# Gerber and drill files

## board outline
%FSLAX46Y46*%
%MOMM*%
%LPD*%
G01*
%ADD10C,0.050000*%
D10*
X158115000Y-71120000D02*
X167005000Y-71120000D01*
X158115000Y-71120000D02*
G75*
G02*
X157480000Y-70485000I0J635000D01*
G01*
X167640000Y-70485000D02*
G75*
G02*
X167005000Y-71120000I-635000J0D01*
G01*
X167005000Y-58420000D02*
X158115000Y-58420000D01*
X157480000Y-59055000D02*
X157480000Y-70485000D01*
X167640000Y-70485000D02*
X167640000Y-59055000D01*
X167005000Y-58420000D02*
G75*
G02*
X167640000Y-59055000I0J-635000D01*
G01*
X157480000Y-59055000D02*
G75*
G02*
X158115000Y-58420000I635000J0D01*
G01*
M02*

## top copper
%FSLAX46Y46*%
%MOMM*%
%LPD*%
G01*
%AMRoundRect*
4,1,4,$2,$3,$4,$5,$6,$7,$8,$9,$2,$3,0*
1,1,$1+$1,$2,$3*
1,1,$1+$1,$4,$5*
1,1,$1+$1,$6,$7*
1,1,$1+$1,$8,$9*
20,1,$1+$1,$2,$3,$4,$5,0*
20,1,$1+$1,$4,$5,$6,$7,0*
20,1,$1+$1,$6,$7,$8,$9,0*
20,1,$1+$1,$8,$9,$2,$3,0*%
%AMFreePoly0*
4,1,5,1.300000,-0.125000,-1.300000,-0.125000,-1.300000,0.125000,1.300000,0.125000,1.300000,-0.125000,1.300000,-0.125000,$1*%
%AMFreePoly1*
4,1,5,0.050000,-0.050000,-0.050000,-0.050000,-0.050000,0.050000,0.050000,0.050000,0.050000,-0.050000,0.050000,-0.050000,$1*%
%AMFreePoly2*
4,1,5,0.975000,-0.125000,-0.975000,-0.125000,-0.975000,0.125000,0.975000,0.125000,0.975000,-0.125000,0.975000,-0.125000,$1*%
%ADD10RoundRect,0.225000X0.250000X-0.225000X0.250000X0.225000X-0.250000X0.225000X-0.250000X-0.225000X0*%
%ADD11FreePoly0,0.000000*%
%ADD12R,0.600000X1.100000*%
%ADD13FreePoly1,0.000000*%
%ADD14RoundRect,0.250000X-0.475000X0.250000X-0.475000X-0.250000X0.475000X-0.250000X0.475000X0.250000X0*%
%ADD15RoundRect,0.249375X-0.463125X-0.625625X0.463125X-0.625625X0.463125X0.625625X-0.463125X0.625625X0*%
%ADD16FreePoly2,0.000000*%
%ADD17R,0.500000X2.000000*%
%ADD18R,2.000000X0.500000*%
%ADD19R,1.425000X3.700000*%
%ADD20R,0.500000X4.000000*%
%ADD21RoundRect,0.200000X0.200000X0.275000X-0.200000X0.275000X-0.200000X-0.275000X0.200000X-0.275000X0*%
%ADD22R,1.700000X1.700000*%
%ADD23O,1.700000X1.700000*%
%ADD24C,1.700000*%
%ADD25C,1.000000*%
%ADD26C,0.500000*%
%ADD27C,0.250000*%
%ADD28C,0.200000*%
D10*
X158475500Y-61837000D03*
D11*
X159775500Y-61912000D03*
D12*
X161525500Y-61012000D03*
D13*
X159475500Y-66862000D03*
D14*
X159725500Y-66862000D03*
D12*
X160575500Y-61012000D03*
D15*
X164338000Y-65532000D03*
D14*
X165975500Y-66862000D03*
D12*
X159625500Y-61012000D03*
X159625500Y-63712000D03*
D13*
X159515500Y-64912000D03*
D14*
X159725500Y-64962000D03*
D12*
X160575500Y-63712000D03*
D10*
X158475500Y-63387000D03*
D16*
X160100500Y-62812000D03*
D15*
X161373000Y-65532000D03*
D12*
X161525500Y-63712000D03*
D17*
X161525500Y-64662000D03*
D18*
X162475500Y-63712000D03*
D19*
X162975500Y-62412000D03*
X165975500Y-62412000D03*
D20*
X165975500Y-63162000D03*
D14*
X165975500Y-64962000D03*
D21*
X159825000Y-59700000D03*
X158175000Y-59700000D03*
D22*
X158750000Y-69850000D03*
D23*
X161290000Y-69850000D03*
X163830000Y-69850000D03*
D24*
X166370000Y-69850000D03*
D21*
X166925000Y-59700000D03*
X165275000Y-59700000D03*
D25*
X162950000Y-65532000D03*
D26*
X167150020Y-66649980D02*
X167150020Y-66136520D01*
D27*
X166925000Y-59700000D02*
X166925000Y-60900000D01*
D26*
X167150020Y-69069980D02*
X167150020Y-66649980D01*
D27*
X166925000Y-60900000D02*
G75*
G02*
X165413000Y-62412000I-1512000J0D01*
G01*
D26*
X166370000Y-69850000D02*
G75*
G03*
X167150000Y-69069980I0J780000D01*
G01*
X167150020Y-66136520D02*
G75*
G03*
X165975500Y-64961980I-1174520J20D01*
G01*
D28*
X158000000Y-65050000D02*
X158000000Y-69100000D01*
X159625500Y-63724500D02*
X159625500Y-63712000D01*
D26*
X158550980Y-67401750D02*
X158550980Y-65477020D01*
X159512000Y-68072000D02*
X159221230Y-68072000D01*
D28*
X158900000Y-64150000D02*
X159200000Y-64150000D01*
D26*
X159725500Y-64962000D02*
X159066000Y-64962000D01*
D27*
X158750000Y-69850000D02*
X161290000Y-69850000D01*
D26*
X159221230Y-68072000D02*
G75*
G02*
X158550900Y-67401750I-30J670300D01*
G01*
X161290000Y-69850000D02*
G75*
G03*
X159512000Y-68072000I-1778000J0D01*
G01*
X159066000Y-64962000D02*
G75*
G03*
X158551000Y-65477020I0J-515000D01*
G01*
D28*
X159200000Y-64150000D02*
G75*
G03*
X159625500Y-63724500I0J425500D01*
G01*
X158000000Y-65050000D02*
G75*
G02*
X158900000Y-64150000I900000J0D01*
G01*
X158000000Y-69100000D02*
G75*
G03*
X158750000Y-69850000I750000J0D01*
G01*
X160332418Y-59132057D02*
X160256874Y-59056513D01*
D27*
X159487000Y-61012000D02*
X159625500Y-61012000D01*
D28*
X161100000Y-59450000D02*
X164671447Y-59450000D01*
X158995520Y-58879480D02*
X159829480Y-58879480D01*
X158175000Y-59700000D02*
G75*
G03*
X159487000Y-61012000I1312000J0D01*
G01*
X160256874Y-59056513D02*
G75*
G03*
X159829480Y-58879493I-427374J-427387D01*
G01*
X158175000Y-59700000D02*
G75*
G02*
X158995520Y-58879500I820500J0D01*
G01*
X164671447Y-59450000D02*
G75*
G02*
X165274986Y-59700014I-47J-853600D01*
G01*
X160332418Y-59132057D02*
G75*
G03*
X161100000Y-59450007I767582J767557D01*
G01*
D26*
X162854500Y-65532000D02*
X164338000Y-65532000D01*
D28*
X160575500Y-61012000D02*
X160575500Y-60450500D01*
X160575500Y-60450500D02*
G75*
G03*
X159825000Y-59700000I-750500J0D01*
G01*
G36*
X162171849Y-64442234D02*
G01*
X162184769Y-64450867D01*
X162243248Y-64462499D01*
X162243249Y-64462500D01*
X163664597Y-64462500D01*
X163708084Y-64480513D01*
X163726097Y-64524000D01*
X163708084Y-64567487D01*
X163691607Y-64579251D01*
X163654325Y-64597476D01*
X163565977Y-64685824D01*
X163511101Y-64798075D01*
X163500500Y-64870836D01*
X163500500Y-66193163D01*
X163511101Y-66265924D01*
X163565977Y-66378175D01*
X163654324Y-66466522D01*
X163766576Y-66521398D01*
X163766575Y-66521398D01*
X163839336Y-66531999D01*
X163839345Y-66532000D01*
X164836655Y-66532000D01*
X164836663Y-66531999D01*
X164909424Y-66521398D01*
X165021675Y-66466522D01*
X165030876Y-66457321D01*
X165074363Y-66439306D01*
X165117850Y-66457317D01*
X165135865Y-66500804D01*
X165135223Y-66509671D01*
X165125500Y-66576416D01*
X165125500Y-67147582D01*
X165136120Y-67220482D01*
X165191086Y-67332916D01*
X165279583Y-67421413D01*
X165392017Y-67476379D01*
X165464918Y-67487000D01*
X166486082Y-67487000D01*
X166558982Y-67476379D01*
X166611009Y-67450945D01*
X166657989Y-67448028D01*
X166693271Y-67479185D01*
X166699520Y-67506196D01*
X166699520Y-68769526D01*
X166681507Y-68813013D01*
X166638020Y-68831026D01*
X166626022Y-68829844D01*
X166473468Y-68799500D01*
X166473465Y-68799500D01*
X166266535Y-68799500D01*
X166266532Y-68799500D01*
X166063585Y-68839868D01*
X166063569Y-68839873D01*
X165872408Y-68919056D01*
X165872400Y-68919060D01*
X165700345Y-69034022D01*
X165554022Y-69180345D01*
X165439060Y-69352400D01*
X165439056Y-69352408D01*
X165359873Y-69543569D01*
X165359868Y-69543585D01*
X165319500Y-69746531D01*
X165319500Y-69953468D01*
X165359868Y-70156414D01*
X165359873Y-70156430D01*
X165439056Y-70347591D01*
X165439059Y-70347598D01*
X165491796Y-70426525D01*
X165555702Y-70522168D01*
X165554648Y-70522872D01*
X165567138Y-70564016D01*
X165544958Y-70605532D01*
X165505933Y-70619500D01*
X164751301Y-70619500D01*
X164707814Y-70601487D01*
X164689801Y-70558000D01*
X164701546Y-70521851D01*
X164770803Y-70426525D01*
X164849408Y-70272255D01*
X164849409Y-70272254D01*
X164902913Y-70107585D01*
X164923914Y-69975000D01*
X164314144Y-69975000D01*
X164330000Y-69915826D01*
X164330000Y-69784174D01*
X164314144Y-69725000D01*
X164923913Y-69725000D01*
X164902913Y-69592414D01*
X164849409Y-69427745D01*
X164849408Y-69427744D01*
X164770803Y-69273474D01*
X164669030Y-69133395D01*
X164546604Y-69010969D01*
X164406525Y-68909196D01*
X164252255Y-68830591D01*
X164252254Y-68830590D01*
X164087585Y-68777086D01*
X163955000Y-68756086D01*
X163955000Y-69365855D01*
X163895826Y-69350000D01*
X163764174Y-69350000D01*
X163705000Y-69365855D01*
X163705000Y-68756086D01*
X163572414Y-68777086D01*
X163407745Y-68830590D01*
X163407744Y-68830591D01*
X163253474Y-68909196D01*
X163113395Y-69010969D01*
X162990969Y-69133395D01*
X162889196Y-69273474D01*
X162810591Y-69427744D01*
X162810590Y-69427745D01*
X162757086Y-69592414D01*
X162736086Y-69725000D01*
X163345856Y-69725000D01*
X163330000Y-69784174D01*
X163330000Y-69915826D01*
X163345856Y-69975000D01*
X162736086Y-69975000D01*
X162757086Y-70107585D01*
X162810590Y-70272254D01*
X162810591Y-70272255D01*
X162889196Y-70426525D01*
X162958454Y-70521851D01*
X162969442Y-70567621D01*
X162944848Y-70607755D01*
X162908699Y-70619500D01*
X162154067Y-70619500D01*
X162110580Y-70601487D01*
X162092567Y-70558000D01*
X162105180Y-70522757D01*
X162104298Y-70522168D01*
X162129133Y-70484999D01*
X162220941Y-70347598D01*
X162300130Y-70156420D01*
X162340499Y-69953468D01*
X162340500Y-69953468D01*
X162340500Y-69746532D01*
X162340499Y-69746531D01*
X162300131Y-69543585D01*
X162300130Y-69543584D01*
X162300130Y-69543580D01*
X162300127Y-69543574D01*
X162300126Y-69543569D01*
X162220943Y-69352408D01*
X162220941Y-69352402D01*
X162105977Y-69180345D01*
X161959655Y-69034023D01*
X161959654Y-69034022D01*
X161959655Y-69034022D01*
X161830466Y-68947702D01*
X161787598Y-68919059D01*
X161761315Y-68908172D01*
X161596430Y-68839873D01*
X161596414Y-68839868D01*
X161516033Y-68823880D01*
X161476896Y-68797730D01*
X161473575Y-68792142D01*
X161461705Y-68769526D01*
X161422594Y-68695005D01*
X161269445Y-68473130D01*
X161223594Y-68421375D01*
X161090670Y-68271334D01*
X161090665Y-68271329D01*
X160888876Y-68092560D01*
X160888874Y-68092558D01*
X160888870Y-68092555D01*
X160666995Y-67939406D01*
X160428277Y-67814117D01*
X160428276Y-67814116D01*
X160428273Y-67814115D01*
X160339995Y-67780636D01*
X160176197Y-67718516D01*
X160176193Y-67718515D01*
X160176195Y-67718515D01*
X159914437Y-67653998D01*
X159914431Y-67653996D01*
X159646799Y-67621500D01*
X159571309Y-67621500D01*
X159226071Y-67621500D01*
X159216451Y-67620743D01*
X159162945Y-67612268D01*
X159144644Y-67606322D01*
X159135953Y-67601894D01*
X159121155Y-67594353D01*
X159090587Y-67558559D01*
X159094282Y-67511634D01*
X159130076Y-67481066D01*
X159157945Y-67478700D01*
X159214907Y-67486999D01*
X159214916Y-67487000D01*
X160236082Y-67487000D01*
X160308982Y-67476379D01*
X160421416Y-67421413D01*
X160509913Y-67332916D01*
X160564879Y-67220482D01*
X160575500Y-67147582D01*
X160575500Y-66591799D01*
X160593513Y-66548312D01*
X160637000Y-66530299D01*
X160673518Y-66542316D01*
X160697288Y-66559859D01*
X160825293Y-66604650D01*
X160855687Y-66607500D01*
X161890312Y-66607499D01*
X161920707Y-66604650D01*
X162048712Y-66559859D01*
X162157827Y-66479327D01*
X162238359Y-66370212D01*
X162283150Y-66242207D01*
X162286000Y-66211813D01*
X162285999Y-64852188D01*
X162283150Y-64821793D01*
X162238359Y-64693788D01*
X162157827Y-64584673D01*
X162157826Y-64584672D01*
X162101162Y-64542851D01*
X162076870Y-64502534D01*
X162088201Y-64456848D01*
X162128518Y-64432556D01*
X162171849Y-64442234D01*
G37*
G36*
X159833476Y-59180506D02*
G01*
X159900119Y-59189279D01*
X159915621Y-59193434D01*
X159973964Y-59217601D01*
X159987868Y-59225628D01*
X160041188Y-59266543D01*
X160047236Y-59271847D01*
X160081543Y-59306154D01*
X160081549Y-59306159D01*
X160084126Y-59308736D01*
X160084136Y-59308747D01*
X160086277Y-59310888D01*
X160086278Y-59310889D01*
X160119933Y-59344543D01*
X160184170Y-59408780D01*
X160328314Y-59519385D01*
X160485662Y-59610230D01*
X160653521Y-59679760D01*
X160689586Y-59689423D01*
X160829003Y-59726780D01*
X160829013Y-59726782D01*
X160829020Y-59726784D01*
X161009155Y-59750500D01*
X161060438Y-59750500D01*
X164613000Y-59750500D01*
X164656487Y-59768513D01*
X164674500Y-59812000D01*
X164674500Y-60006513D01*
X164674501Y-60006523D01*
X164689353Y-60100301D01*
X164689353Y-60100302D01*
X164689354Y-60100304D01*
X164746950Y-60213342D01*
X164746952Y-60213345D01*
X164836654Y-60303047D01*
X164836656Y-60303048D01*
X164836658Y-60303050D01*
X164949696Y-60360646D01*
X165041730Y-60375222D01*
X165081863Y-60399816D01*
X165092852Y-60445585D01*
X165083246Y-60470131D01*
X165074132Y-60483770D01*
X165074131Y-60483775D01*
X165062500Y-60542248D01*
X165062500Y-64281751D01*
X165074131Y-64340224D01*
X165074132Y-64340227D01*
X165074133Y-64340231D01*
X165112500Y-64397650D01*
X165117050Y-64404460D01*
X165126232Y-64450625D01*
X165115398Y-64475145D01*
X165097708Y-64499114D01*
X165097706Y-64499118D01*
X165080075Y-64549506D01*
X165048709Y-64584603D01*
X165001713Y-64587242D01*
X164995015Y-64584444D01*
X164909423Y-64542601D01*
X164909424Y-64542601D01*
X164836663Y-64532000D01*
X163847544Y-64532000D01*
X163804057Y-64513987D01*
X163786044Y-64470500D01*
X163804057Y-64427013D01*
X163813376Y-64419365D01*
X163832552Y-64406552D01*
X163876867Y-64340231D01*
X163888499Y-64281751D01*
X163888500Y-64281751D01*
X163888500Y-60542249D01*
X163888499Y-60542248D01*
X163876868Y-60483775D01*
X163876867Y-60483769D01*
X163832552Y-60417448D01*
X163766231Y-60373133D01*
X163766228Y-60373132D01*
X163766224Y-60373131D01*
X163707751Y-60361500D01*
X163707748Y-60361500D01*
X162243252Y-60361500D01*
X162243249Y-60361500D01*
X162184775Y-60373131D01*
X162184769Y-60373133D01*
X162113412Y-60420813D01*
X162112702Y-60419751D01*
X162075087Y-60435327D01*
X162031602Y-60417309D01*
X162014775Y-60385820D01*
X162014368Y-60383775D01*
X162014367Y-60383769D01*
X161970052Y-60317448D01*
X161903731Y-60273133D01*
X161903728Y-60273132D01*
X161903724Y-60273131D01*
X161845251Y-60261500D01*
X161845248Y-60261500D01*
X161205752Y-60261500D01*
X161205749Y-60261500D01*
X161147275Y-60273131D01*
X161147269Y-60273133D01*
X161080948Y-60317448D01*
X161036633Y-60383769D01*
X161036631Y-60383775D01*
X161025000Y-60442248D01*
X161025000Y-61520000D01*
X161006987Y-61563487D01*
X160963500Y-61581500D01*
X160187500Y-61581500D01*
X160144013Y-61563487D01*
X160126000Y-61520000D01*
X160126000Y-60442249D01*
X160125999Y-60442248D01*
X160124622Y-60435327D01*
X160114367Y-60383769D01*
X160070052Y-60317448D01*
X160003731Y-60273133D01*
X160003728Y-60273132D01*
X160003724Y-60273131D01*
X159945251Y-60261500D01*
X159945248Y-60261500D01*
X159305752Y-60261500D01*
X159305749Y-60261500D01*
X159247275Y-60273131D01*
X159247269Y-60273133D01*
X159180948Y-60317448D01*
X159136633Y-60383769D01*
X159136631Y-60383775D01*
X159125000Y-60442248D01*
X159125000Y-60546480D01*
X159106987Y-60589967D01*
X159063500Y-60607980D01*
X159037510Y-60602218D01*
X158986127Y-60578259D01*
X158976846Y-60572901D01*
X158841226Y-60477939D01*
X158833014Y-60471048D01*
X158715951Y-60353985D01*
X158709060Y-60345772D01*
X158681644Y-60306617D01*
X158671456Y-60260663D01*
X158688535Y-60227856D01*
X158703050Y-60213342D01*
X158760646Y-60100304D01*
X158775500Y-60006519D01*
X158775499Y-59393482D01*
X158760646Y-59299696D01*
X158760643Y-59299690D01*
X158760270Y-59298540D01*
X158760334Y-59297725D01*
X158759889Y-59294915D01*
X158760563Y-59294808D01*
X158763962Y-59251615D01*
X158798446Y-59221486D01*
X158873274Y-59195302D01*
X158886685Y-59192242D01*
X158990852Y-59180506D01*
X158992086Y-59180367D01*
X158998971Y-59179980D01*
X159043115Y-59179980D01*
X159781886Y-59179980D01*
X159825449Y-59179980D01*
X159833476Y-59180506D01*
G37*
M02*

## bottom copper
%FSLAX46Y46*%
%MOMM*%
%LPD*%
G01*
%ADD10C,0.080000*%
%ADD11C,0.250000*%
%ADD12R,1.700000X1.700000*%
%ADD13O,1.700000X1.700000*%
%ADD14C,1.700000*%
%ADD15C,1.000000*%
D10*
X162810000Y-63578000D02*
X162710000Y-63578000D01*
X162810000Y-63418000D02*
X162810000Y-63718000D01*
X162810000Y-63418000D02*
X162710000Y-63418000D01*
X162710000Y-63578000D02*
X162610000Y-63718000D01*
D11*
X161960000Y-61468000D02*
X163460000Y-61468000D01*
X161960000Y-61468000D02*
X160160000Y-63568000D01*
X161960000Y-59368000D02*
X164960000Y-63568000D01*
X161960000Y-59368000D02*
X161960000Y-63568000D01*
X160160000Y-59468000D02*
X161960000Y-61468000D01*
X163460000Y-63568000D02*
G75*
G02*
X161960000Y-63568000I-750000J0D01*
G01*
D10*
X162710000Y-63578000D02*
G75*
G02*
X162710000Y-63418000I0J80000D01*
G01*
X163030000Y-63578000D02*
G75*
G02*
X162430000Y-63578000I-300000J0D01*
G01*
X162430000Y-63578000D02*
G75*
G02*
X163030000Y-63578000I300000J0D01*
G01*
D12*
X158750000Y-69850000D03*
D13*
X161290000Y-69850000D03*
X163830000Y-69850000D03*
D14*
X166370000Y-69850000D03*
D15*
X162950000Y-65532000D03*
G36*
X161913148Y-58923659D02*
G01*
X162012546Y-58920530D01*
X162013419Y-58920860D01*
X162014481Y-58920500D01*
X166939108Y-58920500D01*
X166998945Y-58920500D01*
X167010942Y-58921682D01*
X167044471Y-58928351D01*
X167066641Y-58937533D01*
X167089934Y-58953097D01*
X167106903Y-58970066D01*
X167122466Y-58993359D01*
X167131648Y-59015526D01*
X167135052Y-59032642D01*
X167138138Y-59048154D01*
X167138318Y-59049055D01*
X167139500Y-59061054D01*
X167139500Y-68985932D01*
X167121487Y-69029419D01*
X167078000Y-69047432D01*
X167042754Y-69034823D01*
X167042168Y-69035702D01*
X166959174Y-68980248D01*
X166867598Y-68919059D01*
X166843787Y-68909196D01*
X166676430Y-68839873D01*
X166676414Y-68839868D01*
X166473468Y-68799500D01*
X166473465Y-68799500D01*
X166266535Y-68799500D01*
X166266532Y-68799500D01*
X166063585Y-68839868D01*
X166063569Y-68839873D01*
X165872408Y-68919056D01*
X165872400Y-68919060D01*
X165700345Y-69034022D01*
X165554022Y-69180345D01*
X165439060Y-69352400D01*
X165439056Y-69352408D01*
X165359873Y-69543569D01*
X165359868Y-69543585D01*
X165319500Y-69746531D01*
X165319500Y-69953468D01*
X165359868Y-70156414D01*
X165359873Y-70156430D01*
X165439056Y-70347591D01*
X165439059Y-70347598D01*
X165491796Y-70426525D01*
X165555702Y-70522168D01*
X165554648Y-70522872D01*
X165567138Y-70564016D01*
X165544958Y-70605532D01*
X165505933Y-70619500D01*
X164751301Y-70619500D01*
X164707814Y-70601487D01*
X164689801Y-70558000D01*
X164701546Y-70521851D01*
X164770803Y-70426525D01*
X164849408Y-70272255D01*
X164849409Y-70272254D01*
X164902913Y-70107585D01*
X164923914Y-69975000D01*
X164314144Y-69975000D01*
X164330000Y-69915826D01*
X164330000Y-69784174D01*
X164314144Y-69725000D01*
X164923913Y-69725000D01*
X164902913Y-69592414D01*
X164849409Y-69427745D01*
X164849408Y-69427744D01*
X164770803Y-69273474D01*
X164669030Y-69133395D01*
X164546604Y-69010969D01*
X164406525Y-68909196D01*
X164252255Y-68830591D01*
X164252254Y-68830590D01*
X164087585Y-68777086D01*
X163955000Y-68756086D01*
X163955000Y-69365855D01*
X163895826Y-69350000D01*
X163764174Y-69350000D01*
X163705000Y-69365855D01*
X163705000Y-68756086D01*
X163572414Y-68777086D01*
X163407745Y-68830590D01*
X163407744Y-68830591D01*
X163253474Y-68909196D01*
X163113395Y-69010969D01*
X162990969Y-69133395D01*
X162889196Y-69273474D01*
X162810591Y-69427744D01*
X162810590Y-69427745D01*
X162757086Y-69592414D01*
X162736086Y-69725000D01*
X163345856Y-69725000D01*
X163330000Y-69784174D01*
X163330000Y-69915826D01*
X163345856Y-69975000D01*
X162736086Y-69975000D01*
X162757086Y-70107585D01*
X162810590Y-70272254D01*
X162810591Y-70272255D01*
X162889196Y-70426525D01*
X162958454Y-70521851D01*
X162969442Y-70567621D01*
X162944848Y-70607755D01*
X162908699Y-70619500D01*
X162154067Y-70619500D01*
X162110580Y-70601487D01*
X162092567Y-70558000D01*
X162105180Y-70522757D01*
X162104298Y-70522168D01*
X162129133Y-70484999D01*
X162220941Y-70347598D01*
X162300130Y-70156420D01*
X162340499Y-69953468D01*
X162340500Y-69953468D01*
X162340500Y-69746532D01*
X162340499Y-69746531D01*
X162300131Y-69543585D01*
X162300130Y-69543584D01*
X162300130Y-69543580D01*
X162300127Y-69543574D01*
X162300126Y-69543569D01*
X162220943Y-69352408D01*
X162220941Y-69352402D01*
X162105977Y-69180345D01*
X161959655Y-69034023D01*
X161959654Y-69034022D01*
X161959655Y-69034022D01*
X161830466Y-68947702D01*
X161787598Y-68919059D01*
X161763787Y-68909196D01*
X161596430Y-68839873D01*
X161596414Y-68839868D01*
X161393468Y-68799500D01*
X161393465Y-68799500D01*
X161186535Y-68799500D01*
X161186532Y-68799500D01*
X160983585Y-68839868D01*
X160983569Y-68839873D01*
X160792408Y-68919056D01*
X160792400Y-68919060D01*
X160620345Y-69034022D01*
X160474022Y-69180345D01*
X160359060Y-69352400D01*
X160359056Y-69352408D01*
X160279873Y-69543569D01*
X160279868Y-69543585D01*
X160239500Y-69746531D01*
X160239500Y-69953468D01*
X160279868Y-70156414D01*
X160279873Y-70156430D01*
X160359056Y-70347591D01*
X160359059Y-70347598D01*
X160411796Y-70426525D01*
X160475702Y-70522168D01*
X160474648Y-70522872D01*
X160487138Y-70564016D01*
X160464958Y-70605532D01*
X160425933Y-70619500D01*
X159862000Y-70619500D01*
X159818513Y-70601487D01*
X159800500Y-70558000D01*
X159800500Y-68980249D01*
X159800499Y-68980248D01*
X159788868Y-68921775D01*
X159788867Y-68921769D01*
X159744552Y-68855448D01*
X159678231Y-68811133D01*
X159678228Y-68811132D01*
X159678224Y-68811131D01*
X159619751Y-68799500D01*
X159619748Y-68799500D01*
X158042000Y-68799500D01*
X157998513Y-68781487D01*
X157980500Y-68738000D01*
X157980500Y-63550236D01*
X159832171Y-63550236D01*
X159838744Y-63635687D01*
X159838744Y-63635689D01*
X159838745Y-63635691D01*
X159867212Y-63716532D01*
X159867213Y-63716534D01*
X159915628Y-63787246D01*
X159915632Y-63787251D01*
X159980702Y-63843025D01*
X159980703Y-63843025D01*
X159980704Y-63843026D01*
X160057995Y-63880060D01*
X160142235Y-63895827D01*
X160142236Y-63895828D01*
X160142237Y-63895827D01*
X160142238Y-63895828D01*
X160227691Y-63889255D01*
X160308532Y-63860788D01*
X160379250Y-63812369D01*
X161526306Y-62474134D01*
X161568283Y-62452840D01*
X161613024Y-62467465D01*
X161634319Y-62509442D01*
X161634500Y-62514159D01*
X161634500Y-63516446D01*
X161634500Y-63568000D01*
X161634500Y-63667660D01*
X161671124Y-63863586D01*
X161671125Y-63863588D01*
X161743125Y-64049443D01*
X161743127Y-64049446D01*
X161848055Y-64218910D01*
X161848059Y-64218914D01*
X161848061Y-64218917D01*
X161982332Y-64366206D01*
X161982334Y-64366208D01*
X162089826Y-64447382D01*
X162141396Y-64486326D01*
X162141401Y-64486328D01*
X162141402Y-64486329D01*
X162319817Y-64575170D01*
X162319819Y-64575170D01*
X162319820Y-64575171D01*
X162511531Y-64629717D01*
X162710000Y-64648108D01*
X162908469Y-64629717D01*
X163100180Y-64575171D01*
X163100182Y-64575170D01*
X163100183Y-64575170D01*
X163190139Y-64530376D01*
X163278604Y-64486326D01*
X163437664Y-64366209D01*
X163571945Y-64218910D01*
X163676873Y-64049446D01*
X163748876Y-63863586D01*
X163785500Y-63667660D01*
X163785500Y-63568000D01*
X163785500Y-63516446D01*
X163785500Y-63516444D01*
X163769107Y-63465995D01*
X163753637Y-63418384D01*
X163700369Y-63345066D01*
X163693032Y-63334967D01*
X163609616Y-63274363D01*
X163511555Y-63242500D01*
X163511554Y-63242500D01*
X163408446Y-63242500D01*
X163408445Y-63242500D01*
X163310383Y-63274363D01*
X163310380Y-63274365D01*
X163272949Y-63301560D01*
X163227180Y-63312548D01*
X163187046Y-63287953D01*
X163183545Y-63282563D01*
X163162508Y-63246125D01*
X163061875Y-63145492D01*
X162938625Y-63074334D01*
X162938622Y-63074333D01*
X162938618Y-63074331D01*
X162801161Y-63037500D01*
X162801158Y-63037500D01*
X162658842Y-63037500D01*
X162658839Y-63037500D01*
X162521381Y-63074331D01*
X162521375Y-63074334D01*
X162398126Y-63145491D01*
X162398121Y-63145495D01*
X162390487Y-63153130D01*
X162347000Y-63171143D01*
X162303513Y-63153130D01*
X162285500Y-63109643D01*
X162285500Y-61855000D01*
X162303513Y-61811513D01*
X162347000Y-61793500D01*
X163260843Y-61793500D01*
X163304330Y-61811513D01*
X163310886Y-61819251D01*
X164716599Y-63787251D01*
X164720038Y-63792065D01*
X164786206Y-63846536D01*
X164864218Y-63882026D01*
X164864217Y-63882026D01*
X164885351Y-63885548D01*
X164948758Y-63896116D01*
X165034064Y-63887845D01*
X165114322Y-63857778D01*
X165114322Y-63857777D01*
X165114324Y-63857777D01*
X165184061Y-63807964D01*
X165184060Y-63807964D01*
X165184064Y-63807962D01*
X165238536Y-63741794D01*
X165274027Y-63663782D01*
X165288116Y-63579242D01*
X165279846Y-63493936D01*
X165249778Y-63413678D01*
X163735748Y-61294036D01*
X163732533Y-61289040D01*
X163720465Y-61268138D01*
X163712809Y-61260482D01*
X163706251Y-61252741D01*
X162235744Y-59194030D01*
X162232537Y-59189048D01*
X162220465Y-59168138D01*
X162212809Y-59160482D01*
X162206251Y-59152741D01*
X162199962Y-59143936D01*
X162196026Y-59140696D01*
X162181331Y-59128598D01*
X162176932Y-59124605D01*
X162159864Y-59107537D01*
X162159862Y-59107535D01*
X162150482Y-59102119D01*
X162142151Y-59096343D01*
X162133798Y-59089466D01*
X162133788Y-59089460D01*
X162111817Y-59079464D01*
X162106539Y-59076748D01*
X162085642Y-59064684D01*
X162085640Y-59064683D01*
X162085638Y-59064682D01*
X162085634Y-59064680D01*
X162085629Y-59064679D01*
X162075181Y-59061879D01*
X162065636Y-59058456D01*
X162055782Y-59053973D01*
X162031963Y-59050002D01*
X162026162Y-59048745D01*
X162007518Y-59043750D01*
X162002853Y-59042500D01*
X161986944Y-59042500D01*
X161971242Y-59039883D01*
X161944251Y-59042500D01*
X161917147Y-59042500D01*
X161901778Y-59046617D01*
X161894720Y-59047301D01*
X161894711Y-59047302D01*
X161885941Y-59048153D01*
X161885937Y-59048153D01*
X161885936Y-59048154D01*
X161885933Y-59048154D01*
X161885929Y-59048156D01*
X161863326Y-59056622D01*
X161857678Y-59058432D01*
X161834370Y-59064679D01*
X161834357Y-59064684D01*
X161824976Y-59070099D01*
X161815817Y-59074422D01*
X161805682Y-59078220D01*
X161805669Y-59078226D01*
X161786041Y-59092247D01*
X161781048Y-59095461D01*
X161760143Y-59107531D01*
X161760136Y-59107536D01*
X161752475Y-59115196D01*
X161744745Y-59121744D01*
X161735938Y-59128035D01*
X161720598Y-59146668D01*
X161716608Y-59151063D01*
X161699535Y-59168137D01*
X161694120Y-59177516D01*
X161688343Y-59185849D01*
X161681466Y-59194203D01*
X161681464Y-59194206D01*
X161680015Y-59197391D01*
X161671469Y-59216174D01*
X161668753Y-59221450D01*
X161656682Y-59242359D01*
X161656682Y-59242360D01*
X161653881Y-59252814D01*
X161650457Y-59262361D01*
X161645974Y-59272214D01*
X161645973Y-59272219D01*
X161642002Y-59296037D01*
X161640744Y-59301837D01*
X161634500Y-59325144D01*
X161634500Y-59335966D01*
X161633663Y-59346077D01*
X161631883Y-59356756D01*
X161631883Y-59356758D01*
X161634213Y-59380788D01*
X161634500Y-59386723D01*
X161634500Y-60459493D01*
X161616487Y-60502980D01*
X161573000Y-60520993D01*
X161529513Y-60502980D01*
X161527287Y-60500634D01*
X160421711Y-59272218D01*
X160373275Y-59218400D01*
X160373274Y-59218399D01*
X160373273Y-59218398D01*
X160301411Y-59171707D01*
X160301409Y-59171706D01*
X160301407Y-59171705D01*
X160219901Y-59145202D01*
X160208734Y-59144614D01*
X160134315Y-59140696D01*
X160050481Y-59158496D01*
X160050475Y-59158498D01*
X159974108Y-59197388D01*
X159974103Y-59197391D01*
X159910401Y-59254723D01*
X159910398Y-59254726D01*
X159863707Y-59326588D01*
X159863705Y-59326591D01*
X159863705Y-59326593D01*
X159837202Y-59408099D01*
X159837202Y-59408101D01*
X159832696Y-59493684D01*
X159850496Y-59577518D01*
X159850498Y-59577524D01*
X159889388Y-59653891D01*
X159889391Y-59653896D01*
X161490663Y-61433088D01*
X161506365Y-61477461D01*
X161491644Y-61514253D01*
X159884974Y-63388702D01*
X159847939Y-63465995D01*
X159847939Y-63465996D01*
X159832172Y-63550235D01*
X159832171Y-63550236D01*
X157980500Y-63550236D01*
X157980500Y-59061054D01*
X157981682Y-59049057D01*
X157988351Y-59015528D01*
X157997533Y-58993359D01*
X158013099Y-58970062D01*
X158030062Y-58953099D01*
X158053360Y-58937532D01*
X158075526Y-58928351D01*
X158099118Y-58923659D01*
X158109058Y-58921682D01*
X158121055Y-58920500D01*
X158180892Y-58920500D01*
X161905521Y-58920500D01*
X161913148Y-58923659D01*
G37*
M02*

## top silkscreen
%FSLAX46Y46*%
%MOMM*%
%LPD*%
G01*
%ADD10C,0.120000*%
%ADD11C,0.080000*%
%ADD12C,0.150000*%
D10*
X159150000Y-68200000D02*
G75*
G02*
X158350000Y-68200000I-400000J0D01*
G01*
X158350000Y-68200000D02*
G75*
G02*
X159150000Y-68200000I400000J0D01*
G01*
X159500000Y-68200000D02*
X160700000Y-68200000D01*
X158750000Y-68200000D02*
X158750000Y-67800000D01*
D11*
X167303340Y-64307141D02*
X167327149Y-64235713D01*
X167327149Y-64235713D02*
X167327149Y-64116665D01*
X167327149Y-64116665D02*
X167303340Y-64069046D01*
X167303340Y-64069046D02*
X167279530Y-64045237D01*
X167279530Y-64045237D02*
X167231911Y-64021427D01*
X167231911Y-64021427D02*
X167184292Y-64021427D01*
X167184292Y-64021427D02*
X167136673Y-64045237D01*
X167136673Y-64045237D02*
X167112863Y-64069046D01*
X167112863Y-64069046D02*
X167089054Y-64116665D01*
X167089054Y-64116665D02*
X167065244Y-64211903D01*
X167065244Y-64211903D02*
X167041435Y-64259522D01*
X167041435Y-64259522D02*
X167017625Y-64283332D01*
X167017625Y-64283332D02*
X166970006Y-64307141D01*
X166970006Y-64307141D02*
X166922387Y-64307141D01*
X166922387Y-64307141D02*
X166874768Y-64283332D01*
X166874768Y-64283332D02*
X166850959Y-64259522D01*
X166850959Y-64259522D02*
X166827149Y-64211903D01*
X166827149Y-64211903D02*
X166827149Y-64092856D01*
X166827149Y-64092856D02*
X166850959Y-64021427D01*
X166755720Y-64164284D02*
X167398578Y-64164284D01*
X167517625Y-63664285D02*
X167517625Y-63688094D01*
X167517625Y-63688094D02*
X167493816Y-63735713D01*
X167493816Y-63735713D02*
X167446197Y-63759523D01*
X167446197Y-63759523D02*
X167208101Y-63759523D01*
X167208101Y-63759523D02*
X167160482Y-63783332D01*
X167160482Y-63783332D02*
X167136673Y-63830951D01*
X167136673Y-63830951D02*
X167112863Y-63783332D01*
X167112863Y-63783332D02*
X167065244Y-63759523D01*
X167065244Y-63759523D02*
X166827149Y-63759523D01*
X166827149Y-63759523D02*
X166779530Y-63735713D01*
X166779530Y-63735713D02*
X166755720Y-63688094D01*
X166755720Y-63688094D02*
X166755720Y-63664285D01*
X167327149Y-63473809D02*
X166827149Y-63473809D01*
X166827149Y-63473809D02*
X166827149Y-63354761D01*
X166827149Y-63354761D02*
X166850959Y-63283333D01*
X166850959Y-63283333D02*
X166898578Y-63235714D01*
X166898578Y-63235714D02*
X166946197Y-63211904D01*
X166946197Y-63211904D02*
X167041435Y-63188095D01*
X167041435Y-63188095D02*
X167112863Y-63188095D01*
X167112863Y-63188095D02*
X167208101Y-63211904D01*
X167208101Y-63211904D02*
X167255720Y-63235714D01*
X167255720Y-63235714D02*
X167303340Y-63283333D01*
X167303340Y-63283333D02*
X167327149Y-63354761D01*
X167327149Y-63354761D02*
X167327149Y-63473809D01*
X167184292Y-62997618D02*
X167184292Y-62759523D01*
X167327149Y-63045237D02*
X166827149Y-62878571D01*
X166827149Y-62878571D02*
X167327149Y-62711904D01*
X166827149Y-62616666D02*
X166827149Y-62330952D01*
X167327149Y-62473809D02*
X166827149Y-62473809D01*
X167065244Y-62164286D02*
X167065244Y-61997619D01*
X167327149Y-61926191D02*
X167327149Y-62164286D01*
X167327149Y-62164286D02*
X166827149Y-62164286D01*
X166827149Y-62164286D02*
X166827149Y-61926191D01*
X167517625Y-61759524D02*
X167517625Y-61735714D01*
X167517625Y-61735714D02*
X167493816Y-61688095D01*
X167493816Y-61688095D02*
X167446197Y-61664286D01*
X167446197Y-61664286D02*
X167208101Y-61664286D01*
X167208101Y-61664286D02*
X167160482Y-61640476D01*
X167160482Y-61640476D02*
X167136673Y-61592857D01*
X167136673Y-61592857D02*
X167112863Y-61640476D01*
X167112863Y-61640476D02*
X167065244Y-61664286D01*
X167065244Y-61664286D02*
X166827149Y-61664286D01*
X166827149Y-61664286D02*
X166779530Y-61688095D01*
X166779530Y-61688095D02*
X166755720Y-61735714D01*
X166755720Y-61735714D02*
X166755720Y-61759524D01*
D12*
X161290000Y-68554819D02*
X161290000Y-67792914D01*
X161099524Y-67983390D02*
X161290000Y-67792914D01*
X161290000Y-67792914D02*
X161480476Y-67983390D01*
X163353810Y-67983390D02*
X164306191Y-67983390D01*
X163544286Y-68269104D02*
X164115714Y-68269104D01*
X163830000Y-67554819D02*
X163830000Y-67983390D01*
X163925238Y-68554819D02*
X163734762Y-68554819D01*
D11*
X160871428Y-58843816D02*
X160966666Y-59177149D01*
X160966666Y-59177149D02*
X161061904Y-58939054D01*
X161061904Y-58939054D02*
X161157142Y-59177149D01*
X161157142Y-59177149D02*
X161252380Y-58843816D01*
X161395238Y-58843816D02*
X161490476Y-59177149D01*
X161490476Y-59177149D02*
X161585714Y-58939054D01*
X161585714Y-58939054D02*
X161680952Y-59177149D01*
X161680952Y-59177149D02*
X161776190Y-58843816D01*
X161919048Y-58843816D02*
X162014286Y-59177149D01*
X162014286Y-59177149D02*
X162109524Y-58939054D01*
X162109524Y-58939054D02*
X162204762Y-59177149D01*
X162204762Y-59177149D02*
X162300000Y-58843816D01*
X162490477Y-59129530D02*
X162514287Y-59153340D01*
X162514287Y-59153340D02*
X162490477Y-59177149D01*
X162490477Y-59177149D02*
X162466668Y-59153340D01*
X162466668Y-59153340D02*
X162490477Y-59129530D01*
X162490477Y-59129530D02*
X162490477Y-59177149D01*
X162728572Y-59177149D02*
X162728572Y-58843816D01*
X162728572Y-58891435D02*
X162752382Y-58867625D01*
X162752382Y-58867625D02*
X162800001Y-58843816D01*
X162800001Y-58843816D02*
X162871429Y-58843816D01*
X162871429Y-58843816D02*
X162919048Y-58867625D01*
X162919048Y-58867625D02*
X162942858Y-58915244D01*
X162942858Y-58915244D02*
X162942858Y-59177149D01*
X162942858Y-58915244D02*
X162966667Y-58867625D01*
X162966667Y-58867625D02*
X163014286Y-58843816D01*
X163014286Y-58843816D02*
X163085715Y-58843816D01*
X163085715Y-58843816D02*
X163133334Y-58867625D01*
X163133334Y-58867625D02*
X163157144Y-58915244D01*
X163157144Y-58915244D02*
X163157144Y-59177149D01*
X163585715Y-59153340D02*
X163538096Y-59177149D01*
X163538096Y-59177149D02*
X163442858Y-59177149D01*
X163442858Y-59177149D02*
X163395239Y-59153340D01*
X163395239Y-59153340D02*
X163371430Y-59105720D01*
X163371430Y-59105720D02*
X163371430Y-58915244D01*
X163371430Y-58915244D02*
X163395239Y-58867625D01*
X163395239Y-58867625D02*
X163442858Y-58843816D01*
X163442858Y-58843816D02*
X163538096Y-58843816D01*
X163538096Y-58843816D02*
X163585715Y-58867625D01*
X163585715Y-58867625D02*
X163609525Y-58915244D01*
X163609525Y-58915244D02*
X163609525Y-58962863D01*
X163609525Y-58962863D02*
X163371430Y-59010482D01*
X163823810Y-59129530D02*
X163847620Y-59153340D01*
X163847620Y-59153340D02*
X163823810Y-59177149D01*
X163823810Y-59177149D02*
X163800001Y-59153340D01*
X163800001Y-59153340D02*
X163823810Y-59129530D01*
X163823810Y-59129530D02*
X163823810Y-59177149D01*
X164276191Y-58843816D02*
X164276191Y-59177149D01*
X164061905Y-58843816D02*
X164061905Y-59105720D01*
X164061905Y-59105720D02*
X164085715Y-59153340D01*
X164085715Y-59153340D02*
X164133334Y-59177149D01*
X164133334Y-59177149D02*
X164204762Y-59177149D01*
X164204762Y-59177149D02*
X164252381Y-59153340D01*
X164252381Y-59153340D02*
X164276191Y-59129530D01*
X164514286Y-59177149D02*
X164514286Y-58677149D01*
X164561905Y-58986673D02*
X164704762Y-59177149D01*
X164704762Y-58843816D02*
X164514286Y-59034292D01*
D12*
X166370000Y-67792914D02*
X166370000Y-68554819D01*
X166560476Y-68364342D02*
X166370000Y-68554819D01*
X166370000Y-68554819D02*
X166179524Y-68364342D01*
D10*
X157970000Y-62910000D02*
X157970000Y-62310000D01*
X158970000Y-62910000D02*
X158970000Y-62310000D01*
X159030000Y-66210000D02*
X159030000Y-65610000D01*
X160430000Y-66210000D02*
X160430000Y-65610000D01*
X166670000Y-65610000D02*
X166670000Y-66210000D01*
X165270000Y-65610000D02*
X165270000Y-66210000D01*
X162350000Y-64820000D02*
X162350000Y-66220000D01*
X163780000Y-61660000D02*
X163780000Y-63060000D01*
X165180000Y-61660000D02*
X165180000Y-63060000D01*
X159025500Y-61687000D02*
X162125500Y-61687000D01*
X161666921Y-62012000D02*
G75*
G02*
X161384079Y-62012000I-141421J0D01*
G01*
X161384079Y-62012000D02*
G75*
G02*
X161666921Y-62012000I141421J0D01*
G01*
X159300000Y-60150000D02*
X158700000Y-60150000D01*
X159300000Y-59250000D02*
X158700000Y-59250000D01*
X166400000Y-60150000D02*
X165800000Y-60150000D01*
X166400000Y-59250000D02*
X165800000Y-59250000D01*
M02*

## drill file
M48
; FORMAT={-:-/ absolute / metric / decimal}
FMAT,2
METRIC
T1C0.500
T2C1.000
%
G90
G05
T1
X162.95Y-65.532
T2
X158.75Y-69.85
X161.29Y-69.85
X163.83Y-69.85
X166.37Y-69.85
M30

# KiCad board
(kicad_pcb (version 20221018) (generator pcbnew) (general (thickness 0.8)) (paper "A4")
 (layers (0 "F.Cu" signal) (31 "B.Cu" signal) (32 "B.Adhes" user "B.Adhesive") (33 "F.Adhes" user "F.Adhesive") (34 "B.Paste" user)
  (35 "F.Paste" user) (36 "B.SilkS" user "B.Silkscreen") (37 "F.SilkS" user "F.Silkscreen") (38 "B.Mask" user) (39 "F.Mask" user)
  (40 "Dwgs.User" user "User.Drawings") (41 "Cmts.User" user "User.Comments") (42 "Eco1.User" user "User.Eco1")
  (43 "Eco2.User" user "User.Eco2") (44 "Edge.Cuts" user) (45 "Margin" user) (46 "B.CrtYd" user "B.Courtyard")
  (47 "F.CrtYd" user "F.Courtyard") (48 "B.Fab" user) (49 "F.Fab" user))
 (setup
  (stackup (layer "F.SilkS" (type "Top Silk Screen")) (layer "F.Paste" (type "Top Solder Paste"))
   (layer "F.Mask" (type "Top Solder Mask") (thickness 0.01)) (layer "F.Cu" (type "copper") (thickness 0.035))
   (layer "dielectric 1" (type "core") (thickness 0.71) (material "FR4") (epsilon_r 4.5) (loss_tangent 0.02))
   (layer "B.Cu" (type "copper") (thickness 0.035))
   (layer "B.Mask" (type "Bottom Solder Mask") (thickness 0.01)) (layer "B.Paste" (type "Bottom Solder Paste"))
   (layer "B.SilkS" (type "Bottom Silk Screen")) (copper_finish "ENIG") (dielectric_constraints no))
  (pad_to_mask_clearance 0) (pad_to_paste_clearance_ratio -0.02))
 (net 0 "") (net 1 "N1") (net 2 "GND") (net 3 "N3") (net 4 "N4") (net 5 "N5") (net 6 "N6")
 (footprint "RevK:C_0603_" (layer "F.Cu") (at 158.47 62.61 90)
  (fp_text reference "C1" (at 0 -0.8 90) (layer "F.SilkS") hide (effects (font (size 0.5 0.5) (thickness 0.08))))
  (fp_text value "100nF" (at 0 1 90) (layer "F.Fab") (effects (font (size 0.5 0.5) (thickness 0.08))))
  (fp_line (start -0.3 -0.5) (end 0.3 -0.5) (stroke (width 0.12) (type solid)) (layer "F.SilkS"))
  (fp_line (start -0.3 0.5) (end 0.3 0.5) (stroke (width 0.12) (type solid)) (layer "F.SilkS")))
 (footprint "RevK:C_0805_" (layer "F.Cu") (at 159.73 65.91 90)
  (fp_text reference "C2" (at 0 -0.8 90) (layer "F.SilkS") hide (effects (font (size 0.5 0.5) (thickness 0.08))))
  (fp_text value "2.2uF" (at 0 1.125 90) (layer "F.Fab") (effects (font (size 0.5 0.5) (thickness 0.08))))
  (fp_line (start -0.3 -0.7) (end 0.3 -0.7) (stroke (width 0.12) (type solid)) (layer "F.SilkS"))
  (fp_line (start -0.3 0.7) (end 0.3 0.7) (stroke (width 0.12) (type solid)) (layer "F.SilkS")))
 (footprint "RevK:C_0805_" (layer "F.Cu") (at 165.97 65.91 -90)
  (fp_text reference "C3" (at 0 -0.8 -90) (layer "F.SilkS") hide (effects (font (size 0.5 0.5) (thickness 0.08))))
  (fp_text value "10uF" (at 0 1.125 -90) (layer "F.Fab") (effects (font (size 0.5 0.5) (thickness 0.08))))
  (fp_line (start -0.3 -0.7) (end 0.3 -0.7) (stroke (width 0.12) (type solid)) (layer "F.SilkS"))
  (fp_line (start -0.3 0.7) (end 0.3 0.7) (stroke (width 0.12) (type solid)) (layer "F.SilkS")))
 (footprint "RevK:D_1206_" (layer "F.Cu") (at 162.85 65.52)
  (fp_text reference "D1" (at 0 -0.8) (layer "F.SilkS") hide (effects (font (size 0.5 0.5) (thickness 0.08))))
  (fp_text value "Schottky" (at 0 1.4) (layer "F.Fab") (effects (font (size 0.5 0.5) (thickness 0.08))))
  (fp_line (start -0.5 -0.7) (end -0.5 0.7) (stroke (width 0.12) (type solid)) (layer "F.SilkS")))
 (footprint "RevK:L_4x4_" (layer "F.Cu") (at 164.48 62.36)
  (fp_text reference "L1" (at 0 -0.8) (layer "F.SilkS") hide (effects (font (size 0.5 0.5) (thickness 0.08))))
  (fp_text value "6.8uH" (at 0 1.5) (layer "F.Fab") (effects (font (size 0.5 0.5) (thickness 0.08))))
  (fp_line (start -0.7 -0.7) (end -0.7 0.7) (stroke (width 0.12) (type solid)) (layer "F.SilkS"))
  (fp_line (start 0.7 -0.7) (end 0.7 0.7) (stroke (width 0.12) (type solid)) (layer "F.SilkS")))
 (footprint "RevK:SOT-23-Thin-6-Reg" (layer "F.Cu") (at 160.5755 62.362)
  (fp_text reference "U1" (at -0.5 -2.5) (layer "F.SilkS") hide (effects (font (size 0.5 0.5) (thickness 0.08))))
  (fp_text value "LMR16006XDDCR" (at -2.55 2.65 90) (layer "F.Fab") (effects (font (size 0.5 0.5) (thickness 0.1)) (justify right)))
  (fp_line (start -1.55 -0.675) (end 1.55 -0.675) (stroke (width 0.12) (type solid)) (layer "F.SilkS"))
  (fp_circle (center 0.95 -0.35) (end 1.05 -0.25) (stroke (width 0.12) (type solid)) (fill none) (layer "F.SilkS"))
  (pad "" smd roundrect (at 2.4 -1.1) (size 1.2 1) (layers "F.Paste") (roundrect_rratio 0.25))
  (pad "" smd roundrect (at 2.4 0.05) (size 1.2 1) (layers "F.Paste") (roundrect_rratio 0.25))
  (pad "" smd roundrect (at 2.4 1.2) (size 1.2 1) (layers "F.Paste") (roundrect_rratio 0.25))
  (pad "" smd roundrect (at 5.4 -1.1) (size 1.2 1) (layers "F.Paste") (roundrect_rratio 0.25))
  (pad "" smd roundrect (at 5.4 0.05) (size 1.2 1) (layers "F.Paste") (roundrect_rratio 0.25))
  (pad "" smd roundrect (at 5.4 1.2) (size 1.2 1) (layers "F.Paste") (roundrect_rratio 0.25))
  (pad "1" smd roundrect (at -2.1 -0.525 90) (size 0.9 0.95) (layers "F.Cu" "F.Paste" "F.Mask") (roundrect_rratio 0.25) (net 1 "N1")
   (clearance 0.2))
  (pad "1" smd custom (at -0.8 -0.45) (size 2.6 0.25) (layers "F.Cu") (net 1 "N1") (clearance 0.2) (thermal_bridge_angle 45)
   (options (clearance outline) (anchor rect)) (primitives))
  (pad "1" smd rect (at 0.95 -1.35 90) (size 1.1 0.6) (layers "F.Cu" "F.Paste" "F.Mask") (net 1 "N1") (clearance 0.2))
  (pad "2" smd custom (at -1.1 4.5) (size 0.1 0.1) (layers "F.Cu") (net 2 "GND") (clearance 0.2) (zone_connect 0) (thermal_bridge_angle 45)
   (options (clearance outline) (anchor rect)) (primitives))
  (pad "2" smd roundrect (at -0.85 4.5 270) (size 1 1.45) (layers "F.Cu" "F.Paste" "F.Mask") (roundrect_rratio 0.25) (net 2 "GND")
   (zone_connect 0))
  (pad "2" smd rect (at 0 -1.35 90) (size 1.1 0.6) (layers "F.Cu" "F.Paste" "F.Mask") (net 2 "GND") (clearance 0.2))
  (pad "2" smd roundrect (at 3.7625 3.17) (size 1.425 1.75) (layers "F.Cu" "F.Paste" "F.Mask") (roundrect_rratio 0.175) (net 2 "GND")
   (clearance 0.2) (zone_connect 0))
  (pad "2" smd roundrect (at 5.4 4.5 270) (size 1 1.45) (layers "F.Cu" "F.Paste" "F.Mask") (roundrect_rratio 0.25) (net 2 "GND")
   (zone_connect 0))
  (pad "3" smd rect (at -0.95 -1.35 90) (size 1.1 0.6) (layers "F.Cu" "F.Paste" "F.Mask") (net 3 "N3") (clearance 0.2))
  (pad "4" smd rect (at -0.95 1.35 90) (size 1.1 0.6) (layers "F.Cu" "F.Paste" "F.Mask") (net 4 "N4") (clearance 0.2))
  (pad "5" smd custom (at -1.06 2.55) (size 0.1 0.1) (layers "F.Cu") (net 4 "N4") (zone_connect 0) (thermal_bridge_angle 45)
   (options (clearance outline) (anchor rect)) (primitives))
  (pad "5" smd roundrect (at -0.85 2.6 270) (size 1 1.45) (layers "F.Cu" "F.Paste" "F.Mask") (roundrect_rratio 0.25) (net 4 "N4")
   (clearance 0.2))
  (pad "5" smd rect (at 0 1.35 90) (size 1.1 0.6) (layers "F.Cu" "F.Paste" "F.Mask") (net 4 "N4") (clearance 0.2) (zone_connect 0))
  (pad "6" smd roundrect (at -2.1 1.025 90) (size 0.9 0.95) (layers "F.Cu" "F.Paste" "F.Mask") (roundrect_rratio 0.25) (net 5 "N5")
   (clearance 0.2))
  (pad "6" smd custom (at -0.475 0.45) (size 1.95 0.25) (layers "F.Cu") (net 5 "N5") (clearance 0.2) (thermal_bridge_angle 45)
   (options (clearance outline) (anchor rect)) (primitives))
  (pad "6" smd roundrect (at 0.7975 3.17) (size 1.425 1.75) (layers "F.Cu" "F.Paste" "F.Mask") (roundrect_rratio 0.175) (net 5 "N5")
   (clearance 0.2))
  (pad "6" smd rect (at 0.95 1.35 90) (size 1.1 0.6) (layers "F.Cu" "F.Paste" "F.Mask") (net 5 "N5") (clearance 0.2))
  (pad "6" smd rect (at 0.95 2.3 90) (size 2 0.5) (layers "F.Cu") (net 5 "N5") (clearance 0.2))
  (pad "6" smd rect (at 1.9 1.35) (size 2 0.5) (layers "F.Cu") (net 5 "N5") (clearance 0.2))
  (pad "6" smd rect (at 2.4 0.05 90) (size 3.7 1.425) (layers "F.Cu" "F.Mask") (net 5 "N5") (clearance 0.2))
  (pad "7" smd rect (at 5.4 0.05 90) (size 3.7 1.425) (layers "F.Cu" "F.Mask") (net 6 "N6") (zone_connect 0))
  (pad "7" smd rect (at 5.4 0.8) (size 0.5 4) (layers "F.Cu") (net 6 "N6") (zone_connect 0))
  (pad "7" smd roundrect (at 5.4 2.6 270) (size 1 1.45) (layers "F.Cu" "F.Paste" "F.Mask") (roundrect_rratio 0.25) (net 6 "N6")
   (clearance 0.2) (zone_connect 0)))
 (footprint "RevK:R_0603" (layer "F.Cu") (at 159 59.7 180)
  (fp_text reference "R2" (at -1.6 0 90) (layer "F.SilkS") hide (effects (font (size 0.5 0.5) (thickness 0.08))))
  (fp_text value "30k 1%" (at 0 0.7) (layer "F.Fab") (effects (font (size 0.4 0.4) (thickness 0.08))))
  (fp_line (start -0.3 -0.45) (end 0.3 -0.45) (stroke (width 0.12) (type solid)) (layer "F.SilkS"))
  (fp_line (start -0.3 0.45) (end 0.3 0.45) (stroke (width 0.12) (type solid)) (layer "F.SilkS"))
  (pad "1" smd roundrect (at -0.825 0 180) (size 0.8 0.95) (layers "F.Cu" "F.Paste" "F.Mask") (roundrect_rratio 0.25) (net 2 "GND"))
  (pad "2" smd roundrect (at 0.825 0 180) (size 0.8 0.95) (layers "F.Cu" "F.Paste" "F.Mask") (roundrect_rratio 0.25) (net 3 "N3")))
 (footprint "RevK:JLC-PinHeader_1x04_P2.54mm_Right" (layer "F.Cu") (at 162.56 69.85)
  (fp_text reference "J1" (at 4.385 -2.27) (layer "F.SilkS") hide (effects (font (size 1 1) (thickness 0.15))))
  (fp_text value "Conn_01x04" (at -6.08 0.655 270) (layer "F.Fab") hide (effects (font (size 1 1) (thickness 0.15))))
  (pad "1" thru_hole rect (at -3.81 0 270) (size 1.7 1.7) (drill 1) (layers "*.Cu" "*.Mask") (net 4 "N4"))
  (pad "2" thru_hole oval (at -1.27 0 270) (size 1.7 1.7) (drill 1) (layers "*.Cu" "*.Mask") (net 4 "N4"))
  (pad "3" thru_hole oval (at 1.27 0 270) (size 1.7 1.7) (drill 1) (layers "*.Cu" "*.Mask") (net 2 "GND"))
  (pad "4" thru_hole circle (at 3.81 0 270) (size 1.7 1.7) (drill 1) (layers "*.Cu" "*.Mask") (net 6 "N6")))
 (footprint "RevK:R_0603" (layer "F.Cu") (at 166.1 59.7 180)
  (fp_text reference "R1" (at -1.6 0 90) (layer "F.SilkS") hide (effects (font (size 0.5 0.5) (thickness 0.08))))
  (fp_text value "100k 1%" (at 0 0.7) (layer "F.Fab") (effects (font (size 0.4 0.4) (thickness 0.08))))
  (fp_line (start -0.3 -0.45) (end 0.3 -0.45) (stroke (width 0.12) (type solid)) (layer "F.SilkS"))
  (fp_line (start -0.3 0.45) (end 0.3 0.45) (stroke (width 0.12) (type solid)) (layer "F.SilkS"))
  (pad "1" smd roundrect (at -0.825 0 180) (size 0.8 0.95) (layers "F.Cu" "F.Paste" "F.Mask") (roundrect_rratio 0.25) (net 6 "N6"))
  (pad "2" smd roundrect (at 0.825 0 180) (size 0.8 0.95) (layers "F.Cu" "F.Paste" "F.Mask") (roundrect_rratio 0.25) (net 3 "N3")))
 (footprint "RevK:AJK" (layer "B.Cu") (at 161.96 61.468 180)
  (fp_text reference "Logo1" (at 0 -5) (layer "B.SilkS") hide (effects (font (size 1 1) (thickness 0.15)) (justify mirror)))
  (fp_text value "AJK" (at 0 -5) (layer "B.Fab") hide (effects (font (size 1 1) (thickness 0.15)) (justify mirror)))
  (fp_line (start -0.85 -2.11) (end -0.75 -2.11) (stroke (width 0.08) (type solid)) (layer "B.Cu"))
  (fp_line (start -0.85 -1.95) (end -0.85 -2.25) (stroke (width 0.08) (type solid)) (layer "B.Cu"))
  (fp_line (start -0.85 -1.95) (end -0.75 -1.95) (stroke (width 0.08) (type solid)) (layer "B.Cu"))
  (fp_line (start -0.75 -2.11) (end -0.65 -2.25) (stroke (width 0.08) (type solid)) (layer "B.Cu"))
  (fp_line (start 0 0) (end -1.5 0) (stroke (width 0.25) (type solid)) (layer "B.Cu"))
  (fp_line (start 0 0) (end 1.8 -2.1) (stroke (width 0.25) (type solid)) (layer "B.Cu"))
  (fp_line (start 0 2.1) (end -3 -2.1) (stroke (width 0.25) (type solid)) (layer "B.Cu"))
  (fp_line (start 0 2.1) (end 0 -2.1) (stroke (width 0.25) (type solid)) (layer "B.Cu"))
  (fp_line (start 1.8 2) (end 0 0) (stroke (width 0.25) (type solid)) (layer "B.Cu"))
  (fp_arc (start -1.5 -2.1) (mid -0.75 -2.85) (end 0 -2.1) (stroke (width 0.25) (type solid)) (layer "B.Cu"))
  (fp_arc (start -0.75 -2.11) (mid -0.67 -2.03) (end -0.75 -1.95) (stroke (width 0.08) (type solid)) (layer "B.Cu"))
  (fp_circle (center -0.77 -2.11) (end -0.47 -2.11) (stroke (width 0.08) (type solid)) (fill none) (layer "B.Cu")))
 (gr_circle (center 158.75 68.2) (end 158.75 68.6) (stroke (width 0.12) (type solid)) (fill none) (layer "F.SilkS"))
 (gr_line (start 159.5 68.2) (end 160.7 68.2) (stroke (width 0.12) (type solid)) (layer "F.SilkS"))
 (gr_line (start 158.75 68.2) (end 158.75 67.8) (stroke (width 0.12) (type solid)) (layer "F.SilkS"))
 (gr_line (start 158.115 71.12) (end 167.005 71.12) (stroke (width 0.05) (type solid)) (layer "Edge.Cuts"))
 (gr_arc (start 158.115 71.12) (mid 157.665987 70.934013) (end 157.48 70.485) (stroke (width 0.05) (type solid)) (layer "Edge.Cuts"))
 (gr_arc (start 167.64 70.485) (mid 167.454013 70.934013) (end 167.005 71.12) (stroke (width 0.05) (type solid)) (layer "Edge.Cuts"))
 (gr_line (start 167.005 58.42) (end 158.115 58.42) (stroke (width 0.05) (type solid)) (layer "Edge.Cuts"))
 (gr_line (start 157.48 59.055) (end 157.48 70.485) (stroke (width 0.05) (type solid)) (layer "Edge.Cuts"))
 (gr_line (start 167.64 70.485) (end 167.64 59.055) (stroke (width 0.05) (type solid)) (layer "Edge.Cuts"))
 (gr_arc (start 167.005 58.42) (mid 167.454013 58.605987) (end 167.64 59.055) (stroke (width 0.05) (type solid)) (layer "Edge.Cuts"))
 (gr_arc (start 157.48 59.055) (mid 157.665987 58.605987) (end 158.115 58.42) (stroke (width 0.05) (type solid)) (layer "Edge.Cuts"))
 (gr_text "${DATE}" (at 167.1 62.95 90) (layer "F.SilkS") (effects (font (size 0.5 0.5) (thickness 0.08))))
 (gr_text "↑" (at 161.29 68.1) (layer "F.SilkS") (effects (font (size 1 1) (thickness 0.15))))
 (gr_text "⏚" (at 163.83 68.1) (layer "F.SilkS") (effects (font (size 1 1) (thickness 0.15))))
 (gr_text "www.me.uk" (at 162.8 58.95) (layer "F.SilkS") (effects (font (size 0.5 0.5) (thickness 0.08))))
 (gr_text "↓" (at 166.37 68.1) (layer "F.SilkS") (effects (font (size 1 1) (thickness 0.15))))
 (segment (start 167.15002 66.64998) (end 167.15002 66.13652) (width 0.5) (layer "F.Cu") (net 6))
 (segment (start 166.925 59.7) (end 166.925 60.9) (width 0.25) (layer "F.Cu") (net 6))
 (segment (start 167.15002 69.06998) (end 167.15002 66.64998) (width 0.5) (layer "F.Cu") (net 6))
 (arc (start 166.925 60.9) (mid 166.482145 61.969145) (end 165.413 62.412) (width 0.25) (layer "F.Cu") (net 6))
 (arc (start 166.37 69.85) (mid 166.921557 69.621537) (end 167.15002 69.06998) (width 0.5) (layer "F.Cu") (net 6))
 (arc (start 167.15002 66.13652) (mid 166.806011 65.306009) (end 165.9755 64.962) (width 0.5) (layer "F.Cu") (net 6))
 (segment (start 158 65.05) (end 158 69.1) (width 0.2) (layer "F.Cu") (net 4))
 (segment (start 159.6255 63.7245) (end 159.6255 63.712) (width 0.2) (layer "F.Cu") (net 4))
 (segment (start 158.55098 67.40175) (end 158.55098 65.47702) (width 0.5) (layer "F.Cu") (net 4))
 (segment (start 159.512 68.072) (end 159.22123 68.072) (width 0.5) (layer "F.Cu") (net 4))
 (segment (start 158.9 64.15) (end 159.2 64.15) (width 0.2) (layer "F.Cu") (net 4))
 (segment (start 159.7255 64.962) (end 159.066 64.962) (width 0.5) (layer "F.Cu") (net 4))
 (segment (start 158.75 69.85) (end 161.29 69.85) (width 0.25) (layer "F.Cu") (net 4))
 (arc (start 159.22123 68.072) (mid 158.747292 67.875688) (end 158.55098 67.40175) (width 0.5) (layer "F.Cu") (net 4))
 (arc (start 161.29 69.85) (mid 160.769236 68.592764) (end 159.512 68.072) (width 0.5) (layer "F.Cu") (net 4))
 (arc (start 159.066 64.962) (mid 158.701826 65.112846) (end 158.55098 65.47702) (width 0.5) (layer "F.Cu") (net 4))
 (arc (start 159.2 64.15) (mid 159.500874 64.025374) (end 159.6255 63.7245) (width 0.2) (layer "F.Cu") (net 4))
 (arc (start 158 65.05) (mid 158.263604 64.413604) (end 158.9 64.15) (width 0.2) (layer "F.Cu") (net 4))
 (arc (start 158 69.1) (mid 158.21967 69.63033) (end 158.75 69.85) (width 0.2) (layer "F.Cu") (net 4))
 (segment (start 160.332418 59.132057) (end 160.256874 59.056513) (width 0.2) (layer "F.Cu") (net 3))
 (segment (start 159.487 61.012) (end 159.6255 61.012) (width 0.25) (layer "F.Cu") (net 3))
 (segment (start 161.1 59.45) (end 164.671447 59.45) (width 0.2) (layer "F.Cu") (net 3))
 (segment (start 158.99552 58.87948) (end 159.82948 58.87948) (width 0.2) (layer "F.Cu") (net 3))
 (arc (start 158.175 59.7) (mid 158.559276 60.627724) (end 159.487 61.012) (width 0.2) (layer "F.Cu") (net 3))
 (arc (start 160.256874 59.056513) (mid 160.060784 58.925489) (end 159.82948 58.87948) (width 0.2) (layer "F.Cu") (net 3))
 (arc (start 158.175 59.7) (mid 158.415325 59.119805) (end 158.99552 58.87948) (width 0.2) (layer "F.Cu") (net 3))
 (arc (start 164.671447 59.45) (mid 164.998087 59.514973) (end 165.275 59.7) (width 0.2) (layer "F.Cu") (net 3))
 (arc (start 160.332418 59.132057) (mid 160.684588 59.367369) (end 161.1 59.45) (width 0.2) (layer "F.Cu") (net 3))
 (segment (start 162.8545 65.532) (end 164.338 65.532) (width 0.5) (layer "F.Cu") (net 2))
 (segment (start 160.5755 61.012) (end 160.5755 60.4505) (width 0.2) (layer "F.Cu") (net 2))
 (via (at 162.95 65.532) (size 1) (drill 0.5) (layers "F.Cu" "B.Cu") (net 2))
 (arc (start 160.5755 60.4505) (mid 160.355684 59.919816) (end 159.825 59.7) (width 0.2) (layer "F.Cu") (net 2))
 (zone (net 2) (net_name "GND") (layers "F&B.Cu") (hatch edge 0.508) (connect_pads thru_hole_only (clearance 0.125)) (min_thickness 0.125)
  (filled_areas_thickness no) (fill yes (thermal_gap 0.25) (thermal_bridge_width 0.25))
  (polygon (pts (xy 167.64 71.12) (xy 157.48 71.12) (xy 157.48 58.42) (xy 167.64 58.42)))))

